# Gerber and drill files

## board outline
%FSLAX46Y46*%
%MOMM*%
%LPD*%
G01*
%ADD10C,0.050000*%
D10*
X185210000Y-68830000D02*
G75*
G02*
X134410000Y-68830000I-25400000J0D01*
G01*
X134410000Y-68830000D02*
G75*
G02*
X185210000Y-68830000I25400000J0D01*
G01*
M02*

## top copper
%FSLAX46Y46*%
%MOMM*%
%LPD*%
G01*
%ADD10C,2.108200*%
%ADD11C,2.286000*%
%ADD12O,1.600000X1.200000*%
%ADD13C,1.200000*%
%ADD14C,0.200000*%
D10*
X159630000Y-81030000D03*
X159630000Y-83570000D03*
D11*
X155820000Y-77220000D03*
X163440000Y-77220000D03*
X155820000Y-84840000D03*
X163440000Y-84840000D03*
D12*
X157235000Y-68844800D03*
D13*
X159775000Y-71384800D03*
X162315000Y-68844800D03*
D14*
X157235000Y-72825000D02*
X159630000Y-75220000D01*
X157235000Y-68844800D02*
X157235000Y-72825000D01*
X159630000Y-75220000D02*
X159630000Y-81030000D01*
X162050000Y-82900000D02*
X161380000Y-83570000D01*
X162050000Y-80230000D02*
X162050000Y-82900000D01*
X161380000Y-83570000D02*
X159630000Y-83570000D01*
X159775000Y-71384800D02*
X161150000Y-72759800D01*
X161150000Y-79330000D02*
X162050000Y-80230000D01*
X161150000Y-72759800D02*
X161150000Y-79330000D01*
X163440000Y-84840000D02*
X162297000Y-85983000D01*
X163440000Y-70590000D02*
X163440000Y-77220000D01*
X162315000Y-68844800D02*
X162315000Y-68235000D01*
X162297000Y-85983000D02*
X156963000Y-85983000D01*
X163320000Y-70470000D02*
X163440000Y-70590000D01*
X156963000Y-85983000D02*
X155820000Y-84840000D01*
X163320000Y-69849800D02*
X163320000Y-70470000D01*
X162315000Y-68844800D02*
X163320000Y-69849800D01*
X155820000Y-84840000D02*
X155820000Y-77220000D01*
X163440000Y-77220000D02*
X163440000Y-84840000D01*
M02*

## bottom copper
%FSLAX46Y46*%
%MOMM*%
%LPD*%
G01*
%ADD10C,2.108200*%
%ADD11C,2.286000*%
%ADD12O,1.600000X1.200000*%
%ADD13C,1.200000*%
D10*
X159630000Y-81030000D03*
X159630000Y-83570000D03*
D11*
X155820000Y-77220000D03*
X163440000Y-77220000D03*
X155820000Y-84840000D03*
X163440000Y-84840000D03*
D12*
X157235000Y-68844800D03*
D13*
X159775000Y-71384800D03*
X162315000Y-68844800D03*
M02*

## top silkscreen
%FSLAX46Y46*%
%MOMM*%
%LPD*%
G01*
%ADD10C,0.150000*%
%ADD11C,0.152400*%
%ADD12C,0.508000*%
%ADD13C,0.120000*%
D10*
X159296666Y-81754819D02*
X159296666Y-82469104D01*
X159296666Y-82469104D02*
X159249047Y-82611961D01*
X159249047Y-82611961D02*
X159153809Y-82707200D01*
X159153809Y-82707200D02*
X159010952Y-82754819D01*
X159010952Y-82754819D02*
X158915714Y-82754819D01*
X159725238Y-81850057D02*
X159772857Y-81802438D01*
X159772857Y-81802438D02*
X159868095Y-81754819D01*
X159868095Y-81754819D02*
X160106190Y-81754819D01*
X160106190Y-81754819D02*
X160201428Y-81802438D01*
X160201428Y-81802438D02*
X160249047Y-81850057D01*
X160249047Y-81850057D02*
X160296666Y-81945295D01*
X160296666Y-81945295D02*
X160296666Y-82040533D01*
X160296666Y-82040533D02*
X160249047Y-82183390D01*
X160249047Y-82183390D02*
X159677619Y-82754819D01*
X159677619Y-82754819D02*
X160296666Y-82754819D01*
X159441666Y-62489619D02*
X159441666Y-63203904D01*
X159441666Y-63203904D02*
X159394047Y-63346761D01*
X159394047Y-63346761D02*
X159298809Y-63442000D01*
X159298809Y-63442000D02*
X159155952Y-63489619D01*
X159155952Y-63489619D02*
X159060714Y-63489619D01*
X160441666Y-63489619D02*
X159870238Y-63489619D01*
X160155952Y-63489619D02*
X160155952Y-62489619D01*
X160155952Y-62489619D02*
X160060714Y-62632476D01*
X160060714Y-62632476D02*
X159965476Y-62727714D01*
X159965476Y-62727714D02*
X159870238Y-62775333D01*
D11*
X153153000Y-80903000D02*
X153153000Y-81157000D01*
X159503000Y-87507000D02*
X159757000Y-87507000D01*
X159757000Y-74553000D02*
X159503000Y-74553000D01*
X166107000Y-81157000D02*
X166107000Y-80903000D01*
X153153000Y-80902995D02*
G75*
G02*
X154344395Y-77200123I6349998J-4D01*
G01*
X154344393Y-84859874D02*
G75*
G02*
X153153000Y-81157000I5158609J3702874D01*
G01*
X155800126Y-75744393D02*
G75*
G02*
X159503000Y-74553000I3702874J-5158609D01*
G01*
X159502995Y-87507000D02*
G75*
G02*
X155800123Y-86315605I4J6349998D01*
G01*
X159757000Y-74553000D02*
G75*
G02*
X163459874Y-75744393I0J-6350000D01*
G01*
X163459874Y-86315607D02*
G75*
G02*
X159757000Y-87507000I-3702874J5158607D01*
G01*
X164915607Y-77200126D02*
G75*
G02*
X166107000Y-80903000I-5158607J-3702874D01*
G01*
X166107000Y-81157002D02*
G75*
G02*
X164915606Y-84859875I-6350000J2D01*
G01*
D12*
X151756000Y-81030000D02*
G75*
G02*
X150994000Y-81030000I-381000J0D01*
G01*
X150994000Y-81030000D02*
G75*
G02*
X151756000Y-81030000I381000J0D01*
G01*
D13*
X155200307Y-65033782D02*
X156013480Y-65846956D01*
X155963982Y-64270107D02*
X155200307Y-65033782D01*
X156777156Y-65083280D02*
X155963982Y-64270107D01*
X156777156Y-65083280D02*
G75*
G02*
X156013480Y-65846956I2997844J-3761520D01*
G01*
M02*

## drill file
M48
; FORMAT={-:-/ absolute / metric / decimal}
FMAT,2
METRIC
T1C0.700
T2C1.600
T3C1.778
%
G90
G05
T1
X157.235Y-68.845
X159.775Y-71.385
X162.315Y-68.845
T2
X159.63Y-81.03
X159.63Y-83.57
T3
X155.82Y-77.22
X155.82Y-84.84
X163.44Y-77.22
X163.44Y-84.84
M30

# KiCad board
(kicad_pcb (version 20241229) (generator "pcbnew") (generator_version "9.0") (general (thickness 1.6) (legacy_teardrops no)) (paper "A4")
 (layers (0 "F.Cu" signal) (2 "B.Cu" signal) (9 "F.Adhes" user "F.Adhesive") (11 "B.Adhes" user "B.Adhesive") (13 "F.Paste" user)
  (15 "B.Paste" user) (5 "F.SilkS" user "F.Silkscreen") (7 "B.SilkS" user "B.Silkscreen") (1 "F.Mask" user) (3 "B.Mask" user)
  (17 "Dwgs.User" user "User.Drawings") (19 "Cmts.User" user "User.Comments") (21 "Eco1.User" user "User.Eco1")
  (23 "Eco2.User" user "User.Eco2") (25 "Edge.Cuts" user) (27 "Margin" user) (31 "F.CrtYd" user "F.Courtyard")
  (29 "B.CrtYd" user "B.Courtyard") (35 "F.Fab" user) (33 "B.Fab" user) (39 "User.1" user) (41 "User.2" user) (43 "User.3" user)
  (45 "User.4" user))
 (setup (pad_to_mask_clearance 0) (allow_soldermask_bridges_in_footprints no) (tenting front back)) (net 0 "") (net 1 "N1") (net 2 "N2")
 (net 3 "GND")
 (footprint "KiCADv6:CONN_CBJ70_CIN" (layer "F.Cu") (at 159.63 81.03)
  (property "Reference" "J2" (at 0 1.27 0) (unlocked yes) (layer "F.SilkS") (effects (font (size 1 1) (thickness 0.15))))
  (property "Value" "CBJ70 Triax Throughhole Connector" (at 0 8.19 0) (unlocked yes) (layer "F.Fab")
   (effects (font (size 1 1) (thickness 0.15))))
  (fp_line (start -6.477 -0.127) (end -6.477 0.127) (stroke (width 0.1524) (type solid)) (layer "F.SilkS"))
  (fp_line (start -0.127 6.477) (end 0.127 6.477) (stroke (width 0.1524) (type solid)) (layer "F.SilkS"))
  (fp_line (start 0.127 -6.477) (end -0.127 -6.477) (stroke (width 0.1524) (type solid)) (layer "F.SilkS"))
  (fp_line (start 6.477 0.127) (end 6.477 -0.127) (stroke (width 0.1524) (type solid)) (layer "F.SilkS"))
  (fp_arc (start -6.477 -0.127005) (mid -6.171817 -2.071914) (end -5.285605 -3.829877) (stroke (width 0.1524) (type solid))
   (layer "F.SilkS"))
  (fp_arc (start -5.285607 3.829874) (mid -6.171818 2.07191) (end -6.477 0.127) (stroke (width 0.1524) (type solid)) (layer "F.SilkS"))
  (fp_arc (start -3.829874 -5.285607) (mid -2.07191 -6.171818) (end -0.127 -6.477) (stroke (width 0.1524) (type solid)) (layer "F.SilkS"))
  (fp_arc (start -0.127005 6.477) (mid -2.071914 6.171817) (end -3.829877 5.285605) (stroke (width 0.1524) (type solid)) (layer "F.SilkS"))
  (fp_arc (start 0.127 -6.477) (mid 2.07191 -6.171818) (end 3.829874 -5.285607) (stroke (width 0.1524) (type solid)) (layer "F.SilkS"))
  (fp_arc (start 3.829874 5.285607) (mid 2.07191 6.171818) (end 0.127 6.477) (stroke (width 0.1524) (type solid)) (layer "F.SilkS"))
  (fp_arc (start 5.285607 -3.829874) (mid 6.171818 -2.07191) (end 6.477 -0.127) (stroke (width 0.1524) (type solid)) (layer "F.SilkS"))
  (fp_arc (start 6.477 0.127002) (mid 6.171818 2.071911) (end 5.285606 3.829875) (stroke (width 0.1524) (type solid)) (layer "F.SilkS"))
  (fp_circle (center -8.255 0) (end -7.874 0) (stroke (width 0.508) (type solid)) (fill no) (layer "F.SilkS"))
  (pad "1" thru_hole circle (at 0 0) (size 2.1082 2.1082) (drill 1.6002) (layers "*.Cu" "*.Mask") (remove_unused_layers no) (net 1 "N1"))
  (pad "2" thru_hole circle (at 0 2.54) (size 2.1082 2.1082) (drill 1.6002) (layers "*.Cu" "*.Mask") (remove_unused_layers no) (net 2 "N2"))
  (pad "3" thru_hole circle (at -3.81 -3.81) (size 2.286 2.286) (drill 1.778) (layers "*.Cu" "*.Mask") (remove_unused_layers no)
   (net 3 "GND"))
  (pad "4" thru_hole circle (at 3.81 -3.81) (size 2.286 2.286) (drill 1.778) (layers "*.Cu" "*.Mask" "Dwgs.User") (remove_unused_layers no)
   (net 3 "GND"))
  (pad "5" thru_hole circle (at -3.81 3.81) (size 2.286 2.286) (drill 1.778) (layers "*.Cu" "*.Mask") (remove_unused_layers no)
   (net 3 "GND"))
  (pad "6" thru_hole circle (at 3.81 3.81) (size 2.286 2.286) (drill 1.778) (layers "*.Cu" "*.Mask") (remove_unused_layers no) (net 3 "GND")))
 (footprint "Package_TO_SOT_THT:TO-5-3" (layer "F.Cu") (at 157.235 68.8448)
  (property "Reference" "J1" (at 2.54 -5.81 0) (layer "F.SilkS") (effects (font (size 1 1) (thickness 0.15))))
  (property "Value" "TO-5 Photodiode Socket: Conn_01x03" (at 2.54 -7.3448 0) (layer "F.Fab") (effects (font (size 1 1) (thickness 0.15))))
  (fp_line (start -2.034693 -3.811018) (end -1.22152 -2.997844) (stroke (width 0.12) (type solid)) (layer "F.SilkS"))
  (fp_line (start -1.271018 -4.574693) (end -2.034693 -3.811018) (stroke (width 0.12) (type solid)) (layer "F.SilkS"))
  (fp_line (start -0.457844 -3.76152) (end -1.271018 -4.574693) (stroke (width 0.12) (type solid)) (layer "F.SilkS"))
  (fp_arc (start -0.457844 -3.76152) (mid 5.941184 3.401184) (end -1.22152 -2.997844) (stroke (width 0.12) (type solid)) (layer "F.SilkS"))
  (pad "1" thru_hole oval (at 0 0) (size 1.6 1.2) (drill 0.7) (layers "*.Cu" "*.Mask") (remove_unused_layers no) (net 1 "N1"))
  (pad "2" thru_hole circle (at 2.54 2.54) (size 1.2 1.2) (drill 0.7) (layers "*.Cu" "*.Mask") (remove_unused_layers no) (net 2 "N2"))
  (pad "3" thru_hole circle (at 5.08 0) (size 1.2 1.2) (drill 0.7) (layers "*.Cu" "*.Mask") (remove_unused_layers no) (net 3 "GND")))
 (gr_circle (center 159.81 68.83) (end 185.21 68.83) (stroke (width 0.05) (type solid)) (fill no) (layer "Edge.Cuts"))
 (segment (start 157.235 72.825) (end 159.63 75.22) (width 0.2) (layer "F.Cu") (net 1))
 (segment (start 157.235 68.8448) (end 157.235 72.825) (width 0.2) (layer "F.Cu") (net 1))
 (segment (start 159.63 75.22) (end 159.63 81.03) (width 0.2) (layer "F.Cu") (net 1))
 (segment (start 162.05 82.9) (end 161.38 83.57) (width 0.2) (layer "F.Cu") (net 2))
 (segment (start 162.05 80.23) (end 162.05 82.9) (width 0.2) (layer "F.Cu") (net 2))
 (segment (start 161.38 83.57) (end 159.63 83.57) (width 0.2) (layer "F.Cu") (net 2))
 (segment (start 159.775 71.3848) (end 161.15 72.7598) (width 0.2) (layer "F.Cu") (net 2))
 (segment (start 161.15 79.33) (end 162.05 80.23) (width 0.2) (layer "F.Cu") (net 2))
 (segment (start 161.15 72.7598) (end 161.15 79.33) (width 0.2) (layer "F.Cu") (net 2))
 (segment (start 163.44 84.84) (end 162.297 85.983) (width 0.2) (layer "F.Cu") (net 3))
 (segment (start 163.44 70.59) (end 163.44 77.22) (width 0.2) (layer "F.Cu") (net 3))
 (segment (start 162.315 68.8448) (end 162.315 68.235) (width 0.2) (layer "F.Cu") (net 3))
 (segment (start 162.297 85.983) (end 156.963 85.983) (width 0.2) (layer "F.Cu") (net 3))
 (segment (start 163.32 70.47) (end 163.44 70.59) (width 0.2) (layer "F.Cu") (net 3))
 (segment (start 156.963 85.983) (end 155.82 84.84) (width 0.2) (layer "F.Cu") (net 3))
 (segment (start 163.32 69.8498) (end 163.32 70.47) (width 0.2) (layer "F.Cu") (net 3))
 (segment (start 162.315 68.8448) (end 163.32 69.8498) (width 0.2) (layer "F.Cu") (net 3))
 (segment (start 155.82 84.84) (end 155.82 77.22) (width 0.2) (layer "F.Cu") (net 3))
 (segment (start 163.44 77.22) (end 163.44 84.84) (width 0.2) (layer "F.Cu") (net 3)))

